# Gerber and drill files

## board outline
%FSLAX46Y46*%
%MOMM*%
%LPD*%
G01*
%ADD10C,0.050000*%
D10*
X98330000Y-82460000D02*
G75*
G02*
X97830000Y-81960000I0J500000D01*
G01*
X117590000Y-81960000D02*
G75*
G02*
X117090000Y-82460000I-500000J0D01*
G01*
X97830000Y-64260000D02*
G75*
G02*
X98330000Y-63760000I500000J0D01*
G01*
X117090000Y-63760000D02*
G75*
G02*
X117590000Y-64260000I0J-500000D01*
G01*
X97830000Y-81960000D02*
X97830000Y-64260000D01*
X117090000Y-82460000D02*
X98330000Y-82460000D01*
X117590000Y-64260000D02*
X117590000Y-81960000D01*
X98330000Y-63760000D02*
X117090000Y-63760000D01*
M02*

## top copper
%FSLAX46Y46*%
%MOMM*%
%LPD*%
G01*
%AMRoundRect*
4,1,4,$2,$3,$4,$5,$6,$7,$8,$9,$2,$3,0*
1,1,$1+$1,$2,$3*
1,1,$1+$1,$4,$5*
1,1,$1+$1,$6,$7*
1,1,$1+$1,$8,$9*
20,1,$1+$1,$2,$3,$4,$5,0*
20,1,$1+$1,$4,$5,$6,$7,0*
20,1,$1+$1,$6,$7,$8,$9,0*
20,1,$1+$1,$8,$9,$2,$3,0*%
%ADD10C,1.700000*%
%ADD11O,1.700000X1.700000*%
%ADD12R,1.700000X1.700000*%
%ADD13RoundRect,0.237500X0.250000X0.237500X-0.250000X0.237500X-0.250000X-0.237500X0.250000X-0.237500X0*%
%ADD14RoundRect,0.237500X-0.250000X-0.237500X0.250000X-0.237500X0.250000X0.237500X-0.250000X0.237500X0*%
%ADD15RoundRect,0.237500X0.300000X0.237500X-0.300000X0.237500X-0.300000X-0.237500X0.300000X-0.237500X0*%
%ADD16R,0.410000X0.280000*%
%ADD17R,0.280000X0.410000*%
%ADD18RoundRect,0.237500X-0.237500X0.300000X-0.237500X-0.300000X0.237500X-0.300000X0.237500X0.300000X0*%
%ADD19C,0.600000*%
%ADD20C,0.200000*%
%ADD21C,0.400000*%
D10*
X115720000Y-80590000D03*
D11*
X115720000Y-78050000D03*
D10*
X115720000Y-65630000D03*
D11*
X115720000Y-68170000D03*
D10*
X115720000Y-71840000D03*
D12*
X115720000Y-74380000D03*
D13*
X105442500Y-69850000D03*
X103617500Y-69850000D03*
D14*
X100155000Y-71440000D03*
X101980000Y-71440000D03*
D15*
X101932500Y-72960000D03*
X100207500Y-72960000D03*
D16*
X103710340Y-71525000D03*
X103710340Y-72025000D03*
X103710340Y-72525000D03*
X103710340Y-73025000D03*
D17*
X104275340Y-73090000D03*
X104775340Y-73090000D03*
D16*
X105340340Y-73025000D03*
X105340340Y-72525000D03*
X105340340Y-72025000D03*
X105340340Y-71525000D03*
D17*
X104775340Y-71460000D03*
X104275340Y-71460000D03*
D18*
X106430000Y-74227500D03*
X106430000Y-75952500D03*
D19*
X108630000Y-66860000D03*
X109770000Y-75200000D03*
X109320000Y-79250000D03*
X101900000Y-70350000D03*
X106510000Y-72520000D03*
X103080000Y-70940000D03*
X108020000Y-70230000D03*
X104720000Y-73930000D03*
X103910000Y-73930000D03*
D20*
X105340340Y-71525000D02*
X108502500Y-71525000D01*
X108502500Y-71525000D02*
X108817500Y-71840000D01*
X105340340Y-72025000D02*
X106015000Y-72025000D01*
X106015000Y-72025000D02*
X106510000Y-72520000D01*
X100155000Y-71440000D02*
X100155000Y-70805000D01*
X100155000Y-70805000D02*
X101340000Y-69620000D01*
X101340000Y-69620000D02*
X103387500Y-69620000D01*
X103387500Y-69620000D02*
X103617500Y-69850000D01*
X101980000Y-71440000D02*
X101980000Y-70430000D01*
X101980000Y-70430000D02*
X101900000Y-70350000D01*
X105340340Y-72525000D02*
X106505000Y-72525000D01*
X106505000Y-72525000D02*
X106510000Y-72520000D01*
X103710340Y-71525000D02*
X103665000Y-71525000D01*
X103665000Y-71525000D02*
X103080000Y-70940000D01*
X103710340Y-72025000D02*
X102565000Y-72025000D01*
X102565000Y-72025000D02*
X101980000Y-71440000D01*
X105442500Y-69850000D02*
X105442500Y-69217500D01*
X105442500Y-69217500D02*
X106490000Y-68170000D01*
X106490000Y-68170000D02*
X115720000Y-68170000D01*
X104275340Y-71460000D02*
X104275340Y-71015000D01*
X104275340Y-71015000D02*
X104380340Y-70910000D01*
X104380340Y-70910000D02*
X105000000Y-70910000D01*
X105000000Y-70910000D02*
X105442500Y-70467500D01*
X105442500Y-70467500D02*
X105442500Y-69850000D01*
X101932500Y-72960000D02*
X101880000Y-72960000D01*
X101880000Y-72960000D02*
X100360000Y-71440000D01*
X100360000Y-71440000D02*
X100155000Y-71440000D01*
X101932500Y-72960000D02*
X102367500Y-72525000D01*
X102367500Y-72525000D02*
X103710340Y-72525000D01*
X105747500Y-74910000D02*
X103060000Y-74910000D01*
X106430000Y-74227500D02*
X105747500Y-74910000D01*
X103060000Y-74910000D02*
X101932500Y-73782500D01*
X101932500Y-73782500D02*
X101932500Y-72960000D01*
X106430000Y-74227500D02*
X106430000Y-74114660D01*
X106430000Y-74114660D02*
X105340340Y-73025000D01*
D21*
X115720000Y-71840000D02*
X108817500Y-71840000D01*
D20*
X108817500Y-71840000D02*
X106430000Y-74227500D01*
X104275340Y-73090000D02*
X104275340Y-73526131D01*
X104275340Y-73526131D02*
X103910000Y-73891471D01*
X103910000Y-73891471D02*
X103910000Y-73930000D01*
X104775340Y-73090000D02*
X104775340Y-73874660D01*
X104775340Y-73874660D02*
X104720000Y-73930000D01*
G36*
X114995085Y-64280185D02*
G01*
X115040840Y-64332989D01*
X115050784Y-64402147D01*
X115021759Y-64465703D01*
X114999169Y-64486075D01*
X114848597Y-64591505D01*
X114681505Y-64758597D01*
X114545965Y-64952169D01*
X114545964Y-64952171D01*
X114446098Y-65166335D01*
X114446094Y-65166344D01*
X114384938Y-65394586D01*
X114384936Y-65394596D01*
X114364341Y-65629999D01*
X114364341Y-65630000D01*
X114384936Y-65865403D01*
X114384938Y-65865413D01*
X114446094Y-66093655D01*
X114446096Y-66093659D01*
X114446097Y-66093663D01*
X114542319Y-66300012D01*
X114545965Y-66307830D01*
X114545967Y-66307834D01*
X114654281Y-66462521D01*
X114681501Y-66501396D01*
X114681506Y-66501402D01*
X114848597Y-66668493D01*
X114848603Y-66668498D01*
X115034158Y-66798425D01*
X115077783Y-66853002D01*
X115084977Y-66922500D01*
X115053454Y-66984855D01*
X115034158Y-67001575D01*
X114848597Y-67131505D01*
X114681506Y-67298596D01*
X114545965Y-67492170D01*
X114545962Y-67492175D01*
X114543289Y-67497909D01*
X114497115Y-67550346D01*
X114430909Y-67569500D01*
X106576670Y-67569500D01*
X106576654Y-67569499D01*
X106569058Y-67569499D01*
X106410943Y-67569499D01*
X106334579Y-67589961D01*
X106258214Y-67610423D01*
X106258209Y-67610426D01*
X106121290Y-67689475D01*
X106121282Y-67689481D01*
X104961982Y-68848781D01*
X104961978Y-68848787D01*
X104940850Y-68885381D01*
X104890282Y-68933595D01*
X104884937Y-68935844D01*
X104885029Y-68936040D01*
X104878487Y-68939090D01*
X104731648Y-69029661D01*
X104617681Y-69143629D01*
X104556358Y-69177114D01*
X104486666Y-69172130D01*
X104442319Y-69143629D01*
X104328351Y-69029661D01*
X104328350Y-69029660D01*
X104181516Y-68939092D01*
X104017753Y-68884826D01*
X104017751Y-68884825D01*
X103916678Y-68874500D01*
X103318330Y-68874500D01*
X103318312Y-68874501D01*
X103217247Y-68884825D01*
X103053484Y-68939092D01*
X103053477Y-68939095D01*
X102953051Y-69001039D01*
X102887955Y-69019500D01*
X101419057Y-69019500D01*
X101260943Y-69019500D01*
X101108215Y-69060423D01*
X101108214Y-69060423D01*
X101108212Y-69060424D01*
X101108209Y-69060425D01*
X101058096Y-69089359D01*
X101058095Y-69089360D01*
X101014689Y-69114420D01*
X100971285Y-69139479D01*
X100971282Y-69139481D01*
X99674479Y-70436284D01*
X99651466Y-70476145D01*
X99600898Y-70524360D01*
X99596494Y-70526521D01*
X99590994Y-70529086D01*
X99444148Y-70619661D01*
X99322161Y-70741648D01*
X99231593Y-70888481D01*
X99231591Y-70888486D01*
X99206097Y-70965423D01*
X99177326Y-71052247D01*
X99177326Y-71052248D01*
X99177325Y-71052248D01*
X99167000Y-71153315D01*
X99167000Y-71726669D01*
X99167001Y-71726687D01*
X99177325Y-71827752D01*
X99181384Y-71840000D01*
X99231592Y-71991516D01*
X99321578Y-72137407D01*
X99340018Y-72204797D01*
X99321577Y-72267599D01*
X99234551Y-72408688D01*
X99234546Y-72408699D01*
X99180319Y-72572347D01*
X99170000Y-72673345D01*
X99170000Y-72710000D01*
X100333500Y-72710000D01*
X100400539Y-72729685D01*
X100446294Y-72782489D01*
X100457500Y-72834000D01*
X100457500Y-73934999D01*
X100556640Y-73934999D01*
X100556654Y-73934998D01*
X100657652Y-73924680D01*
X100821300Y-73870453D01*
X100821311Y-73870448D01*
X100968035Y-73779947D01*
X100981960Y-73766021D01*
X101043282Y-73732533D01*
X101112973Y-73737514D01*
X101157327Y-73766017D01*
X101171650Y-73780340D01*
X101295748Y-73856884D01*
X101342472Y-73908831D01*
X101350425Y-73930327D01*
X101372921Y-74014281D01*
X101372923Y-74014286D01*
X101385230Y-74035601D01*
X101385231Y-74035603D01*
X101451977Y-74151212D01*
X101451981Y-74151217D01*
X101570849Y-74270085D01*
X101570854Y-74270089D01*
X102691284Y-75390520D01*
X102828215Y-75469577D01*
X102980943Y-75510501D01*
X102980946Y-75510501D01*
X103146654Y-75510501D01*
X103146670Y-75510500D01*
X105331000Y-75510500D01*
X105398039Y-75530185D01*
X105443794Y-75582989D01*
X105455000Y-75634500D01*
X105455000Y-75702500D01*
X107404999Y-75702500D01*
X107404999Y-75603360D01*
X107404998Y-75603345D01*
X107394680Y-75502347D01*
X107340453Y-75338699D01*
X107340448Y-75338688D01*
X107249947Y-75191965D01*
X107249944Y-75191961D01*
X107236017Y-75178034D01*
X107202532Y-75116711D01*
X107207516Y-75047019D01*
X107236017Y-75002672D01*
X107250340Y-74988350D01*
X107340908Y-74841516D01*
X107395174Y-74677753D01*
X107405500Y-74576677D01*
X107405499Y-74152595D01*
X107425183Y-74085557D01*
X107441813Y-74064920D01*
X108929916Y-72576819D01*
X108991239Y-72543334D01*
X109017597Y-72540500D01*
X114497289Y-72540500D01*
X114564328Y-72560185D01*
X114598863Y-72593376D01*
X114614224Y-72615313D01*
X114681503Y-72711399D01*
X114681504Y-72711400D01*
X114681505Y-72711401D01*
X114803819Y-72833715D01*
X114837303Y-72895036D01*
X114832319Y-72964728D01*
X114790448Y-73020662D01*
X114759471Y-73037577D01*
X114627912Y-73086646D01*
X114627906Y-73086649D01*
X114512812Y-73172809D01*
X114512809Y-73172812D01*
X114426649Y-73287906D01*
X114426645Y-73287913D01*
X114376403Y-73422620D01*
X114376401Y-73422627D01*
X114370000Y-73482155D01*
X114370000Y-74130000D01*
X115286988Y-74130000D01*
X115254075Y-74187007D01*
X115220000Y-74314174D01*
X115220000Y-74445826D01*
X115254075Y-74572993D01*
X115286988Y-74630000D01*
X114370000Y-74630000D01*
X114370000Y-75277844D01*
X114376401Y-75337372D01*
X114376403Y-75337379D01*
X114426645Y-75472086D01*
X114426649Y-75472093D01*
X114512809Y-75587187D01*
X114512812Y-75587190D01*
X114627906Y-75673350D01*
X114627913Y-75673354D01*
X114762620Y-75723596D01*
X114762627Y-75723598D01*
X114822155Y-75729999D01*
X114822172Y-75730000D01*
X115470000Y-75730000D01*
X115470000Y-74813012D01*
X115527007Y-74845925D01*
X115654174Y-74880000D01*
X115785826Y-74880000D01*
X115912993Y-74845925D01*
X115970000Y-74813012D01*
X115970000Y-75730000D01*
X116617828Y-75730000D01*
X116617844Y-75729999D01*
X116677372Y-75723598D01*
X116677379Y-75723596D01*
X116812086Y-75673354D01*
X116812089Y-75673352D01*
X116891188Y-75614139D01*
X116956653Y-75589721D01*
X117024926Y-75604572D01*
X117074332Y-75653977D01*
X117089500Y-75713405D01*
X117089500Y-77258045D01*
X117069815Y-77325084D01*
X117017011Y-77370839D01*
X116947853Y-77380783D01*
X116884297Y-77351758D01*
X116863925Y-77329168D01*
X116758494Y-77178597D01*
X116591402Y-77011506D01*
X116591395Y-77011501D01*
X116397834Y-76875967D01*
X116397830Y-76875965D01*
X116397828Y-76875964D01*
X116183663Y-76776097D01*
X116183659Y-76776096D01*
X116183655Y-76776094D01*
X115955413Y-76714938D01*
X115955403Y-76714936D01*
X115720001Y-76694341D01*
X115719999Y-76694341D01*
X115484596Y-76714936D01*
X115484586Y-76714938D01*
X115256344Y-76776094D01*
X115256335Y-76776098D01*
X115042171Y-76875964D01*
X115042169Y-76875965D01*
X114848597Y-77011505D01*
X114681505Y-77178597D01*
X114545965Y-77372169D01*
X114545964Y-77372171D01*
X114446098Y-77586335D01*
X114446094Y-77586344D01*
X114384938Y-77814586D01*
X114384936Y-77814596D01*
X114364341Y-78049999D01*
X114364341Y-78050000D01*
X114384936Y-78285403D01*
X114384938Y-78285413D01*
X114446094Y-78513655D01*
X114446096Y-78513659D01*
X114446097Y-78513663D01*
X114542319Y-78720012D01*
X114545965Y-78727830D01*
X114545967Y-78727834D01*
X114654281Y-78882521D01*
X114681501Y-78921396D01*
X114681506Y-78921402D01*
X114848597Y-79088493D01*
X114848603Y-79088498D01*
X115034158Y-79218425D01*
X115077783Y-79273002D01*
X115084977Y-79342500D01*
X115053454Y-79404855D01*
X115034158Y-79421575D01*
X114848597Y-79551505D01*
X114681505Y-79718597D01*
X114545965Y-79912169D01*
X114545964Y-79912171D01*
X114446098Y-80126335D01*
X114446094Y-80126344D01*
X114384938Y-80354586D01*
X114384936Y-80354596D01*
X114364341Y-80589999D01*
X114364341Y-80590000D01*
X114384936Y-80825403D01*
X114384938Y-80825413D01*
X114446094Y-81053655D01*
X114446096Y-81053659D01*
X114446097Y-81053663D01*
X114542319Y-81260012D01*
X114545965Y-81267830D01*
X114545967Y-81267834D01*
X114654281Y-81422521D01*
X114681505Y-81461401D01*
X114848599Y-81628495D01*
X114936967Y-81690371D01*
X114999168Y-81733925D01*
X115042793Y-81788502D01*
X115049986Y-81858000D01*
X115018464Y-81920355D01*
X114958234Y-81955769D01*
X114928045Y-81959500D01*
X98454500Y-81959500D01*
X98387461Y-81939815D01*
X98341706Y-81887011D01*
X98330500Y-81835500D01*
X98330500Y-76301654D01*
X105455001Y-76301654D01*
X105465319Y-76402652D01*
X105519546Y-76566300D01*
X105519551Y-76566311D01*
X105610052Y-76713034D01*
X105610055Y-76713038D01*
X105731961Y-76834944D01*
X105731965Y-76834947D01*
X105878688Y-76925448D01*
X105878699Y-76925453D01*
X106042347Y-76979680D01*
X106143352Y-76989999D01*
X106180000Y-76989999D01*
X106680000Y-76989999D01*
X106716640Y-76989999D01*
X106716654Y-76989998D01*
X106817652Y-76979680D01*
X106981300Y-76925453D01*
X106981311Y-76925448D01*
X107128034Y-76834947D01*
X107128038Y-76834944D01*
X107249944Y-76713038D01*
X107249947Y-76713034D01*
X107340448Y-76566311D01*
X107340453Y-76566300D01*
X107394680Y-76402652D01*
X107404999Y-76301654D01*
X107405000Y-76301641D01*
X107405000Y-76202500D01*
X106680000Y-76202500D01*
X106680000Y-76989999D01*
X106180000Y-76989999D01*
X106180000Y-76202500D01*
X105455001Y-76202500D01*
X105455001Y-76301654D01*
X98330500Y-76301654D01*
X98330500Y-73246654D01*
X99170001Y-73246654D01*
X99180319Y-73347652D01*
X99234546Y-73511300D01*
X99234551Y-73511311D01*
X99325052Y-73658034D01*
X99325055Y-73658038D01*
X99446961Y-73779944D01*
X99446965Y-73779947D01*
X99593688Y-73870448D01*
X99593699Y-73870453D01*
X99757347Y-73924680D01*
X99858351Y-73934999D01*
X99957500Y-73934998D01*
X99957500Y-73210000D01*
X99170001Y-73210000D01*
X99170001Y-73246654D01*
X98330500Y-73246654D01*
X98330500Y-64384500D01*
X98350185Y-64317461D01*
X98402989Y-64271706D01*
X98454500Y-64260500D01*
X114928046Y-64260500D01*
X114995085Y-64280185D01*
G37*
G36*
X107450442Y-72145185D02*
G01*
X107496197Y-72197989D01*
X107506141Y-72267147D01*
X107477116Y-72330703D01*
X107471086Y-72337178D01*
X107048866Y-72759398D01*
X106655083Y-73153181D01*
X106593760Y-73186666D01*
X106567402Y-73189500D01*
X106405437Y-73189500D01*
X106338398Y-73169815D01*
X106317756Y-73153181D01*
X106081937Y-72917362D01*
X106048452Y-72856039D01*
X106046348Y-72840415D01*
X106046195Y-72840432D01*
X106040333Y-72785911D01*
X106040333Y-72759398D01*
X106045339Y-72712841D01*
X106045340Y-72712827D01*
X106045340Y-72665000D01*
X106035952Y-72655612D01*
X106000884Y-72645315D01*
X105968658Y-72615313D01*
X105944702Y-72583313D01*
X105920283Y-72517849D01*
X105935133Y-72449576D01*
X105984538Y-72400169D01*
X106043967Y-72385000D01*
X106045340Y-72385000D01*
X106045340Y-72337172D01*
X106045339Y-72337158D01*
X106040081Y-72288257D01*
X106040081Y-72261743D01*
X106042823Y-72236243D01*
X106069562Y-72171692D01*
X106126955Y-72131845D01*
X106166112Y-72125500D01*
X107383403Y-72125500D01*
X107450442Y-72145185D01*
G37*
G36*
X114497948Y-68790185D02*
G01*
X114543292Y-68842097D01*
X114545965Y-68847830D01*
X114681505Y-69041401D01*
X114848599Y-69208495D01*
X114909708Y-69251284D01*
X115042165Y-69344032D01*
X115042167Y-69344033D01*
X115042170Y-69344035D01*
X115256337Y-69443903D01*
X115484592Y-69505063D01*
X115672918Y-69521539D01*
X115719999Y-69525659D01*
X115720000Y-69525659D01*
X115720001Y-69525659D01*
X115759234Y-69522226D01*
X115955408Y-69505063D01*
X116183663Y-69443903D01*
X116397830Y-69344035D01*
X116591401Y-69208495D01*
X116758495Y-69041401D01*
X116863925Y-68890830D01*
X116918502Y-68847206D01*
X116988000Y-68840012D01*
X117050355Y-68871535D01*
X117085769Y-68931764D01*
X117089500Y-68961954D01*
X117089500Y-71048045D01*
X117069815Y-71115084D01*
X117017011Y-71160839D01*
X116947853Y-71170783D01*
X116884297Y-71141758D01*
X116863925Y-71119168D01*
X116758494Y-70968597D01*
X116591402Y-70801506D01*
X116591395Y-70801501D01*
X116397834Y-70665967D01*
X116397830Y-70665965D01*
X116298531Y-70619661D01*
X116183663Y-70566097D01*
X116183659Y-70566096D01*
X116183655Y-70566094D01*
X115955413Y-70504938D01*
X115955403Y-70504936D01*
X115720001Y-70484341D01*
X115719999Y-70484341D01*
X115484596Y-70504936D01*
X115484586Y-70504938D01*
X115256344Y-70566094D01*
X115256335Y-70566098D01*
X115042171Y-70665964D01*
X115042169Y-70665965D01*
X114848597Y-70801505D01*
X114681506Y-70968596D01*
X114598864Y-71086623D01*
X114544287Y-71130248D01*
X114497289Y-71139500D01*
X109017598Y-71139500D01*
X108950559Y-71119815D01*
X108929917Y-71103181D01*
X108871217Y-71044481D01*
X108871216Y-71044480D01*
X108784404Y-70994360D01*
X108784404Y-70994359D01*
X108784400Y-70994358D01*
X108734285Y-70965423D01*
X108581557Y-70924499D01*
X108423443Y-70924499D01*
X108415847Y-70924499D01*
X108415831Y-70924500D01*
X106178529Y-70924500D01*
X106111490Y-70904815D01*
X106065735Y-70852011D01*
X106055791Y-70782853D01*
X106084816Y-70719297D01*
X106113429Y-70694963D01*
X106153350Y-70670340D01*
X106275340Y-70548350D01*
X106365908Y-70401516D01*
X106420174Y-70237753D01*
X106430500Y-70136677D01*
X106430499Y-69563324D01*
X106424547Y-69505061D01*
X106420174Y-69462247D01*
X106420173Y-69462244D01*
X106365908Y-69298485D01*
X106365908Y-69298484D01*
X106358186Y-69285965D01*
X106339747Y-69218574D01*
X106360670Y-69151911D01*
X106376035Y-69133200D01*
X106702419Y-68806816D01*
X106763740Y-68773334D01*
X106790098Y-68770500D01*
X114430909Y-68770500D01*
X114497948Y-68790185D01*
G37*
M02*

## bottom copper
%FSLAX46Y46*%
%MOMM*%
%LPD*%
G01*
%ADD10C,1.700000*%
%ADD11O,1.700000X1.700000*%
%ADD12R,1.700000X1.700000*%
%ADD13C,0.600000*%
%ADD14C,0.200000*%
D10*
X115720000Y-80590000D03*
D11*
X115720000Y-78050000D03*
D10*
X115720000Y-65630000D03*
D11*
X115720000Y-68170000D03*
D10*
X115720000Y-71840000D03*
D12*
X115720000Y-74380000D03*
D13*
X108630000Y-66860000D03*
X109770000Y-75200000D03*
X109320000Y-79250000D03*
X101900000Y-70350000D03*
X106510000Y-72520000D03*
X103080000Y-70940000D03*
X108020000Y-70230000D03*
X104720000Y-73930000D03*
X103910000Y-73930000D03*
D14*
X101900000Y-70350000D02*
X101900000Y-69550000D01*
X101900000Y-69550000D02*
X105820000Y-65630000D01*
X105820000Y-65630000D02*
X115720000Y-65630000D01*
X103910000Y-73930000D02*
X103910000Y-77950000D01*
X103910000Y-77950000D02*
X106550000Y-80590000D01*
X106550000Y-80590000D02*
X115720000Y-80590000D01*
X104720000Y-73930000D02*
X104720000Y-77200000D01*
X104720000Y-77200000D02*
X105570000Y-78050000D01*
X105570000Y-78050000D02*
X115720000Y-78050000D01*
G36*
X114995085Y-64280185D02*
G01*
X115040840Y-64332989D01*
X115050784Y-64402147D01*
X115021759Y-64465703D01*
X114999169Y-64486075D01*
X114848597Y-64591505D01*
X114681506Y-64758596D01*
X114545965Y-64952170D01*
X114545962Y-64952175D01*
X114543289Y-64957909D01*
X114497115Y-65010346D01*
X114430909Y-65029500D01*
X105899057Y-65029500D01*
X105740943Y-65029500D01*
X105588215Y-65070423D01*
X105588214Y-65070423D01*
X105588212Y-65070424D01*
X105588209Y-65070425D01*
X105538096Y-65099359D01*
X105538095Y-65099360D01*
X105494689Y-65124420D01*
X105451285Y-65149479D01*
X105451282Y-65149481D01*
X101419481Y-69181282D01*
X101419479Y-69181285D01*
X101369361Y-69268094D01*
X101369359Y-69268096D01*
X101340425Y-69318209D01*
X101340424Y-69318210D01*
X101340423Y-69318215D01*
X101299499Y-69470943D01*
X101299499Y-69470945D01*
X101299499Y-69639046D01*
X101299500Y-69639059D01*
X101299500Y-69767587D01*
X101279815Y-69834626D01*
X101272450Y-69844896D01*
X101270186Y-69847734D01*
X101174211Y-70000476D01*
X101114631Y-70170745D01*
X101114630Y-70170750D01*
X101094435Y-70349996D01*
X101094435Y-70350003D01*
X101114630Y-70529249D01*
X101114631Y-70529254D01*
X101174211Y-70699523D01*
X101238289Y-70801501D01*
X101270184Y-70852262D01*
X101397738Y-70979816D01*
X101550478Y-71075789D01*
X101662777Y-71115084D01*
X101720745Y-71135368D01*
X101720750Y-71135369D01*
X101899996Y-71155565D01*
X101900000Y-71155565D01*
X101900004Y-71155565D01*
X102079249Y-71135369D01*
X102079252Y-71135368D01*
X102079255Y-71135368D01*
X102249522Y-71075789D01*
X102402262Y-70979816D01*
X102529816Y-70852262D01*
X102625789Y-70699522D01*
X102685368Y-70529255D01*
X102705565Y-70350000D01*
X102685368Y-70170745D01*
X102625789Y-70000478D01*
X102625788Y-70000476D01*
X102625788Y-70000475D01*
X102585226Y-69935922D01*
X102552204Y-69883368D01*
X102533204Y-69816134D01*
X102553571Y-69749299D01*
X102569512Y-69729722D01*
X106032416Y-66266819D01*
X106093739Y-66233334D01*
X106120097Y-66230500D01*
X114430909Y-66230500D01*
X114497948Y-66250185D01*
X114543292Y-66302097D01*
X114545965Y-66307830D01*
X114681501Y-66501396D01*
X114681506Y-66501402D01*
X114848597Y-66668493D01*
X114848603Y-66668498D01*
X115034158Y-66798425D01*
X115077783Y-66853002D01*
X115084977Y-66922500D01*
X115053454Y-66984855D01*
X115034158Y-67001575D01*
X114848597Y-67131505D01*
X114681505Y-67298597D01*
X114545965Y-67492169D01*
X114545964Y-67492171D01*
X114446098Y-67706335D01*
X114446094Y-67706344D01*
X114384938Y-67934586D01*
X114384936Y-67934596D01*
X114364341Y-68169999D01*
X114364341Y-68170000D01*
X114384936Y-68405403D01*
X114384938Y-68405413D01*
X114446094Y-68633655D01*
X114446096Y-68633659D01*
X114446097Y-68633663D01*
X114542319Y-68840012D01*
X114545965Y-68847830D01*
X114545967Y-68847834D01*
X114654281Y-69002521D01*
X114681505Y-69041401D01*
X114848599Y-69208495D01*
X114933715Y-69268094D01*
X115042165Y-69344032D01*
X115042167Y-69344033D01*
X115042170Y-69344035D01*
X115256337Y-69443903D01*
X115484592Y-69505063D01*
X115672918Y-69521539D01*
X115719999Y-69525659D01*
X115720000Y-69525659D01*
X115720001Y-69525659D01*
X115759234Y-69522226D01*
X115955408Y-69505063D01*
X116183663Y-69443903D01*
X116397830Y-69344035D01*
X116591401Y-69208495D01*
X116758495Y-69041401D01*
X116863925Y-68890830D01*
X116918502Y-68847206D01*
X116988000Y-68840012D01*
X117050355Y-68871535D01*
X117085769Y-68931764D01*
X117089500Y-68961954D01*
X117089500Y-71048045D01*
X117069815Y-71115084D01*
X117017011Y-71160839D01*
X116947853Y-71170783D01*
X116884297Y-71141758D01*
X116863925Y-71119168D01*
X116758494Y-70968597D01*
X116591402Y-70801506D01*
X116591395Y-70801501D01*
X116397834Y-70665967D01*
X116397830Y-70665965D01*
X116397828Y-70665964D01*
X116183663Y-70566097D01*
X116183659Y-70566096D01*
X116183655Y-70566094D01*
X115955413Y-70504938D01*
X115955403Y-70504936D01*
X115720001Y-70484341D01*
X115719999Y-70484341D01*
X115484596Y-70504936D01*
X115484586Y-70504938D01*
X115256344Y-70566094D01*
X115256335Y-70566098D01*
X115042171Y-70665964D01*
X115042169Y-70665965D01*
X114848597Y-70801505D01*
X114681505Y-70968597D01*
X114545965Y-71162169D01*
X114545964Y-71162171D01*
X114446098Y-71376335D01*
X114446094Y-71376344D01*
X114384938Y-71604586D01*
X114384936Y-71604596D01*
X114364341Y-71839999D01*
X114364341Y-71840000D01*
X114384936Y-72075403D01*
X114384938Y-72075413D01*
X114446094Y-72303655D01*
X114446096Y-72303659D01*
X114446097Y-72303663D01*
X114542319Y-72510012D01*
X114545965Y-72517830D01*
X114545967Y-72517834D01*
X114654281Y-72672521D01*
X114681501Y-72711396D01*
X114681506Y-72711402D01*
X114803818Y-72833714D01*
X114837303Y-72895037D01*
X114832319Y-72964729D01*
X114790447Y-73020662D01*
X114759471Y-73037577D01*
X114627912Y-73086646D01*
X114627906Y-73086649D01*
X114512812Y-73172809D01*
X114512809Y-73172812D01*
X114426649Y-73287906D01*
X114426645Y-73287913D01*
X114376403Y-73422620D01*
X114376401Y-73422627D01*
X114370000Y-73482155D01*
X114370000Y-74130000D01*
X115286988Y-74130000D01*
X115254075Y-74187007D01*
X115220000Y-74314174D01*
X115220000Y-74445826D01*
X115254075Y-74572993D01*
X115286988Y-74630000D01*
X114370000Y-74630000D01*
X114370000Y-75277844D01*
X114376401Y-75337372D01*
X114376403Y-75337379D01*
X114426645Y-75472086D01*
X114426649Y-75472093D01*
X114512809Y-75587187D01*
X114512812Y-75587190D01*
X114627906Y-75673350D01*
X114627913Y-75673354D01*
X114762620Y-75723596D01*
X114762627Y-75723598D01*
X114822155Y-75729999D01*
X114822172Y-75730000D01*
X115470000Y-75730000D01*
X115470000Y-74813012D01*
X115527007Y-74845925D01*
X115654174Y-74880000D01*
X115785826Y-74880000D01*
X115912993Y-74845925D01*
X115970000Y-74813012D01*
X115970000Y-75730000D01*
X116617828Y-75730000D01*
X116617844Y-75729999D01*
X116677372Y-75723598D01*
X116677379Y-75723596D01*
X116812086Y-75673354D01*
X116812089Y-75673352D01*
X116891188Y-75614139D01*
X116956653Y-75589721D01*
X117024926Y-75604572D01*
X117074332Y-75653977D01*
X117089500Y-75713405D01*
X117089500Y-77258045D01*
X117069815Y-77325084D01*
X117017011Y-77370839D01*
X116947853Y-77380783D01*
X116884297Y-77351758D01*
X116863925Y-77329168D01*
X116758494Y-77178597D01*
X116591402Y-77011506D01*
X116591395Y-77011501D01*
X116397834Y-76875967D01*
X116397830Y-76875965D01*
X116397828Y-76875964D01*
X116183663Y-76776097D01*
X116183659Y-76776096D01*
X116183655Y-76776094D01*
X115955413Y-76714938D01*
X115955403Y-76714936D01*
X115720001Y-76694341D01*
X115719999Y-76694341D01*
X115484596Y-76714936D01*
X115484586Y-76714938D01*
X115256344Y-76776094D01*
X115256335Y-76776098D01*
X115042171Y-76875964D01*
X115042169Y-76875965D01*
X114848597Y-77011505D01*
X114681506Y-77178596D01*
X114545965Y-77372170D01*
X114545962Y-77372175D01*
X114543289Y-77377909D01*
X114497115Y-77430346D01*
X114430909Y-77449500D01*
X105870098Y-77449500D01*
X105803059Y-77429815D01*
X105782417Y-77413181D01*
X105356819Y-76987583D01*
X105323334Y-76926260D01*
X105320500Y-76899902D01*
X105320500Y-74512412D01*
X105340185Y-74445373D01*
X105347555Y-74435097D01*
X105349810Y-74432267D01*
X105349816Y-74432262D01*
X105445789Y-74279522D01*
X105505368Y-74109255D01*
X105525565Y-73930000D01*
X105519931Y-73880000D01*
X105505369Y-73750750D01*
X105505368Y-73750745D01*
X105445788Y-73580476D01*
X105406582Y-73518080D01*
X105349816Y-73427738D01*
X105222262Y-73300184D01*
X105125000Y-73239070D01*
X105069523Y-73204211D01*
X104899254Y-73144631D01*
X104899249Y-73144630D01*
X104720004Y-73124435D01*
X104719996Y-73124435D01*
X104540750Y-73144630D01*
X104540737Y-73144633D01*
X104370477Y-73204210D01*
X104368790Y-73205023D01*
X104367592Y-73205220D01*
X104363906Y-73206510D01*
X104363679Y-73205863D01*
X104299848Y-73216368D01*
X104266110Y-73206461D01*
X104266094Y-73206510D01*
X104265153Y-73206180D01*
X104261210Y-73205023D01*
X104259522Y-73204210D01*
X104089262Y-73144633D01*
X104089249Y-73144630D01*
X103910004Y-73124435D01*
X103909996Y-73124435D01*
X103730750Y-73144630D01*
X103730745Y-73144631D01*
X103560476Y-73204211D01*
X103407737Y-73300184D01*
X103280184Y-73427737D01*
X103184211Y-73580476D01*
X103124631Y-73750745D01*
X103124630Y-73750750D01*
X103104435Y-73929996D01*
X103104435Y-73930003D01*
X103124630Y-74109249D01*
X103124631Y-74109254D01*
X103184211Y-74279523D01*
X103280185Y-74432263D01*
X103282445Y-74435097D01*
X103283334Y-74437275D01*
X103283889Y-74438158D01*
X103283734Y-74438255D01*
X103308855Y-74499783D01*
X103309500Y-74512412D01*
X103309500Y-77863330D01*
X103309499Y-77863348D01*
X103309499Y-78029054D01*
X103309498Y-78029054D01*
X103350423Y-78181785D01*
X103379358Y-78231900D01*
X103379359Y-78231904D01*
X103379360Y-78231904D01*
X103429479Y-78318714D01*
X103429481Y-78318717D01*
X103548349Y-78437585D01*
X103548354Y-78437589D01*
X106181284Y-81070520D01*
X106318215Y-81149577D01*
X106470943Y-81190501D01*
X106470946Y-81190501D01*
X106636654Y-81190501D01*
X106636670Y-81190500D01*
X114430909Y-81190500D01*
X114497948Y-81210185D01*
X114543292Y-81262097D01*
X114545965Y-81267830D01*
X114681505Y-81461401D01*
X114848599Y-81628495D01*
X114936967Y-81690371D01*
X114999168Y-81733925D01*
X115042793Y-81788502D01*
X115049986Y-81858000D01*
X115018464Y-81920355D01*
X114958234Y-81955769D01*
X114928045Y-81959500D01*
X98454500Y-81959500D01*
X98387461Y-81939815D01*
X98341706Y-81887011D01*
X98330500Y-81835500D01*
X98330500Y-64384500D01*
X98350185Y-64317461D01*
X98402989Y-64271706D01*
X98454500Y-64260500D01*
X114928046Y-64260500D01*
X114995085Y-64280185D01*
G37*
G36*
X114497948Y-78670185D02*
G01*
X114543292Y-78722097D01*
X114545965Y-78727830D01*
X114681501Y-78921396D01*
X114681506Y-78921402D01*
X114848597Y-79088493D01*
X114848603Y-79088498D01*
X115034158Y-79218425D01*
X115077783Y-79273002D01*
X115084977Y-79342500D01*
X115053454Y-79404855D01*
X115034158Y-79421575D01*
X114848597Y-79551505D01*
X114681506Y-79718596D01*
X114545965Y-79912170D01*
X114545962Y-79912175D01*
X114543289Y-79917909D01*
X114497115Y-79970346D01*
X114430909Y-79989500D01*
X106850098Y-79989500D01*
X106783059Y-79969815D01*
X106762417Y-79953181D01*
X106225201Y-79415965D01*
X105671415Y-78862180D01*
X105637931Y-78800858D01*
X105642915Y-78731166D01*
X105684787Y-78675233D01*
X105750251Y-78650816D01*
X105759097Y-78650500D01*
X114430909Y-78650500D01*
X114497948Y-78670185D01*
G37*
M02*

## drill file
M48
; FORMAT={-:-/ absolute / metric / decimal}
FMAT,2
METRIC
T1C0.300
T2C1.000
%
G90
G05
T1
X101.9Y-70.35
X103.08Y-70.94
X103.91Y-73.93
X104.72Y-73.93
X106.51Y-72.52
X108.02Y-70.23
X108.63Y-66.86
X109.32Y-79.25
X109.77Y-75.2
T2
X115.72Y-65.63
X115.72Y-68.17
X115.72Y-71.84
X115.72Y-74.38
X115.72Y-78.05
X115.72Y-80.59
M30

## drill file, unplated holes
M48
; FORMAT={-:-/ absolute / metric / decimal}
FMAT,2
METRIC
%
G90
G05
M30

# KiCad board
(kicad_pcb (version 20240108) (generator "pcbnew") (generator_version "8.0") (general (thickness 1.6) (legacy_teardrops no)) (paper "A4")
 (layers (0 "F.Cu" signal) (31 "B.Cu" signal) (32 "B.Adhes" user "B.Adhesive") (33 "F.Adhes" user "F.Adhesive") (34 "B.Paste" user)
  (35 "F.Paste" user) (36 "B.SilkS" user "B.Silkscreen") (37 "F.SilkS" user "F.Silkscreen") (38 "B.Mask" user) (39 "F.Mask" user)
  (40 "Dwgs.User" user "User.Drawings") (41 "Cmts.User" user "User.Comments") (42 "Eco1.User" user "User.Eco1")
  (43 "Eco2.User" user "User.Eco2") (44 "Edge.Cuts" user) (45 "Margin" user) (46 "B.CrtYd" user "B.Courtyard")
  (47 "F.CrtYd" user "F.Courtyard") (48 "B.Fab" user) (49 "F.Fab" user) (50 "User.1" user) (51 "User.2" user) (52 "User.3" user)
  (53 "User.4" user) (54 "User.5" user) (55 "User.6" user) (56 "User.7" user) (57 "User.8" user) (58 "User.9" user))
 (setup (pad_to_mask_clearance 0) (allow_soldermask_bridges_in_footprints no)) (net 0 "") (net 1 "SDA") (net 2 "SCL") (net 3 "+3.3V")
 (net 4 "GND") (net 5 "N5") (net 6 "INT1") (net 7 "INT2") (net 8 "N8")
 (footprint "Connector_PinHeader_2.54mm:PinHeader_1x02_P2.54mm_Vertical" (layer "F.Cu") (at 115.72 65.63)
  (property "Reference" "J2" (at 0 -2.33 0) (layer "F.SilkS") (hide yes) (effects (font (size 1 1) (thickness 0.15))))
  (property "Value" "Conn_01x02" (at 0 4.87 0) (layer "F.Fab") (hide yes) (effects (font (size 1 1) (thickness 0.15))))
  (pad "1" thru_hole circle (at 0 0) (size 1.7 1.7) (drill 1) (layers "*.Cu" "*.Mask") (remove_unused_layers no) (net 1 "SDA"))
  (pad "2" thru_hole oval (at 0 2.54) (size 1.7 1.7) (drill 1) (layers "*.Cu" "*.Mask") (remove_unused_layers no) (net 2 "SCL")))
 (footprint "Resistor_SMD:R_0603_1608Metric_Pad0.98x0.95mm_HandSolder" (layer "F.Cu") (at 104.53 69.85 180)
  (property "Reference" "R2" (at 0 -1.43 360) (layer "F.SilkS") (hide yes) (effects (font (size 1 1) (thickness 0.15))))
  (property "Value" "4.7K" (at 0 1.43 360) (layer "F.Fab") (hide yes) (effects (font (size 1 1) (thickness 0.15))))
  (pad "1" smd roundrect (at -0.9125 0 180) (size 0.975 0.95) (layers "F.Cu" "F.Paste" "F.Mask") (roundrect_rratio 0.25) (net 2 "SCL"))
  (pad "2" smd roundrect (at 0.9125 0 180) (size 0.975 0.95) (layers "F.Cu" "F.Paste" "F.Mask") (roundrect_rratio 0.25) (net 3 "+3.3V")))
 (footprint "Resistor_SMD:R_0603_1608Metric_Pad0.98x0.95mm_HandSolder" (layer "F.Cu") (at 101.0675 71.44)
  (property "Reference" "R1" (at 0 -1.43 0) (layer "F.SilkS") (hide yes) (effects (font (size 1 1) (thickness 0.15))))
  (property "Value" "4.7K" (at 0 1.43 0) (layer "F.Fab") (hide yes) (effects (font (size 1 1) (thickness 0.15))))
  (pad "1" smd roundrect (at -0.9125 0) (size 0.975 0.95) (layers "F.Cu" "F.Paste" "F.Mask") (roundrect_rratio 0.25) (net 3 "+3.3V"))
  (pad "2" smd roundrect (at 0.9125 0) (size 0.975 0.95) (layers "F.Cu" "F.Paste" "F.Mask") (roundrect_rratio 0.25) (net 1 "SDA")))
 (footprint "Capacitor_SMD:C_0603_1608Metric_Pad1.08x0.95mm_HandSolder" (layer "F.Cu") (at 101.07 72.96 180)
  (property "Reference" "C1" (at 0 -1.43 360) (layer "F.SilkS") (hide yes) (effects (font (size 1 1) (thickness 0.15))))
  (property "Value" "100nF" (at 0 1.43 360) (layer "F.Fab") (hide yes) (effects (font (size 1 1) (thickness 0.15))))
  (pad "1" smd roundrect (at -0.8625 0 180) (size 1.075 0.95) (layers "F.Cu" "F.Paste" "F.Mask") (roundrect_rratio 0.25) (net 3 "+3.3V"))
  (pad "2" smd roundrect (at 0.8625 0 180) (size 1.075 0.95) (layers "F.Cu" "F.Paste" "F.Mask") (roundrect_rratio 0.25) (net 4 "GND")))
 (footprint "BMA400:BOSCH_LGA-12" (layer "F.Cu") (at 104.52534 72.275)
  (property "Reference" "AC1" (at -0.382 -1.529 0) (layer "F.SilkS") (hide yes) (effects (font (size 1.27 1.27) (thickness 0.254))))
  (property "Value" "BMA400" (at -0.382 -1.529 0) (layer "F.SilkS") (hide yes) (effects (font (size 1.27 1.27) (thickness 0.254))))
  (pad "1" smd rect (at -0.815 -0.75 90) (size 0.28 0.41) (layers "F.Cu" "F.Paste" "F.Mask") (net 4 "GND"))
  (pad "2" smd rect (at -0.815 -0.25 90) (size 0.28 0.41) (layers "F.Cu" "F.Paste" "F.Mask") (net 1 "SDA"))
  (pad "3" smd rect (at -0.815 0.25 90) (size 0.28 0.41) (layers "F.Cu" "F.Paste" "F.Mask") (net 3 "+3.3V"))
  (pad "4" smd rect (at -0.815 0.75 90) (size 0.28 0.41) (layers "F.Cu" "F.Paste" "F.Mask") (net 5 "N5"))
  (pad "5" smd rect (at -0.25 0.815) (size 0.28 0.41) (layers "F.Cu" "F.Paste" "F.Mask") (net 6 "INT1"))
  (pad "6" smd rect (at 0.25 0.815) (size 0.28 0.41) (layers "F.Cu" "F.Paste" "F.Mask") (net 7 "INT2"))
  (pad "7" smd rect (at 0.815 0.75 90) (size 0.28 0.41) (layers "F.Cu" "F.Paste" "F.Mask") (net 3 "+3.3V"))
  (pad "8" smd rect (at 0.815 0.25 90) (size 0.28 0.41) (layers "F.Cu" "F.Paste" "F.Mask") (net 4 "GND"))
  (pad "9" smd rect (at 0.815 -0.25 90) (size 0.28 0.41) (layers "F.Cu" "F.Paste" "F.Mask") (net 4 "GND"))
  (pad "10" smd rect (at 0.815 -0.75 90) (size 0.28 0.41) (layers "F.Cu" "F.Paste" "F.Mask") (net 3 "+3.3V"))
  (pad "11" smd rect (at 0.25 -0.815) (size 0.28 0.41) (layers "F.Cu" "F.Paste" "F.Mask") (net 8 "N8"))
  (pad "12" smd rect (at -0.25 -0.815) (size 0.28 0.41) (layers "F.Cu" "F.Paste" "F.Mask") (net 2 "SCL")))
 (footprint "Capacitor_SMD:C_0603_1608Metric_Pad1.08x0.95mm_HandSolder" (layer "F.Cu") (at 106.43 75.09 -90)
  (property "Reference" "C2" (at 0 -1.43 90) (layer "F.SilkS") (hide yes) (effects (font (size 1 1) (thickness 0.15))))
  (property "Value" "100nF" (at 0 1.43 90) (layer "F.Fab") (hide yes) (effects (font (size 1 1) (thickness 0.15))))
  (pad "1" smd roundrect (at -0.8625 0 270) (size 1.075 0.95) (layers "F.Cu" "F.Paste" "F.Mask") (roundrect_rratio 0.25) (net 3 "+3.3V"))
  (pad "2" smd roundrect (at 0.8625 0 270) (size 1.075 0.95) (layers "F.Cu" "F.Paste" "F.Mask") (roundrect_rratio 0.25) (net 4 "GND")))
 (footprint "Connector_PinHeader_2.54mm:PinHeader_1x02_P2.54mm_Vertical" (layer "F.Cu") (at 115.72 71.84)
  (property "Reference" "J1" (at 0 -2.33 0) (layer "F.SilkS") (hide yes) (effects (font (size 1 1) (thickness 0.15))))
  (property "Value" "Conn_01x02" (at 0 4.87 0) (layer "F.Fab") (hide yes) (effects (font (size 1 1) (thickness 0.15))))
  (pad "1" thru_hole circle (at 0 0) (size 1.7 1.7) (drill 1) (layers "*.Cu" "*.Mask") (remove_unused_layers no) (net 3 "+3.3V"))
  (pad "2" thru_hole rect (at 0 2.54) (size 1.7 1.7) (drill 1) (layers "*.Cu" "*.Mask") (remove_unused_layers no) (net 4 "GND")))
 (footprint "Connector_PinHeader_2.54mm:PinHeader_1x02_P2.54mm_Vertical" (layer "F.Cu") (at 115.72 80.59 180)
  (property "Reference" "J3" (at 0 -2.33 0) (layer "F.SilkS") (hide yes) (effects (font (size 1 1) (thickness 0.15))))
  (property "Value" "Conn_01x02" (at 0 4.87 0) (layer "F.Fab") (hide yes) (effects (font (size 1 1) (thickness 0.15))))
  (pad "1" thru_hole circle (at 0 0 180) (size 1.7 1.7) (drill 1) (layers "*.Cu" "*.Mask") (remove_unused_layers no) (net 6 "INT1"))
  (pad "2" thru_hole oval (at 0 2.54 180) (size 1.7 1.7) (drill 1) (layers "*.Cu" "*.Mask") (remove_unused_layers no) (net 7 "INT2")))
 (gr_arc (start 117.09 63.76) (mid 117.443553 63.906447) (end 117.59 64.26) (stroke (width 0.05) (type default)) (layer "Edge.Cuts"))
 (gr_line (start 117.09 82.46) (end 98.33 82.46) (stroke (width 0.05) (type default)) (layer "Edge.Cuts"))
 (gr_arc (start 97.83 64.26) (mid 97.976447 63.906447) (end 98.33 63.76) (stroke (width 0.05) (type default)) (layer "Edge.Cuts"))
 (gr_arc (start 98.33 82.46) (mid 97.976447 82.313553) (end 97.83 81.96) (stroke (width 0.05) (type default)) (layer "Edge.Cuts"))
 (gr_arc (start 117.59 81.96) (mid 117.443553 82.313553) (end 117.09 82.46) (stroke (width 0.05) (type default)) (layer "Edge.Cuts"))
 (gr_line (start 117.59 64.26) (end 117.59 81.96) (stroke (width 0.05) (type default)) (layer "Edge.Cuts"))
 (gr_line (start 97.83 81.96) (end 97.83 64.26) (stroke (width 0.05) (type default)) (layer "Edge.Cuts"))
 (gr_line (start 98.33 63.76) (end 117.09 63.76) (stroke (width 0.05) (type default)) (layer "Edge.Cuts"))
 (segment (start 101.34 69.62) (end 103.3875 69.62) (width 0.2) (layer "F.Cu") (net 3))
 (segment (start 100.155 71.44) (end 100.155 70.805) (width 0.2) (layer "F.Cu") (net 3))
 (segment (start 108.5025 71.525) (end 108.8175 71.84) (width 0.2) (layer "F.Cu") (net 3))
 (segment (start 101.9325 73.7825) (end 101.9325 72.96) (width 0.2) (layer "F.Cu") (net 3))
 (segment (start 108.8175 71.84) (end 106.43 74.2275) (width 0.2) (layer "F.Cu") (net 3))
 (segment (start 106.43 74.2275) (end 106.43 74.11466) (width 0.2) (layer "F.Cu") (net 3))
 (segment (start 106.43 74.2275) (end 105.7475 74.91) (width 0.2) (layer "F.Cu") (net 3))
 (segment (start 102.3675 72.525) (end 103.71034 72.525) (width 0.2) (layer "F.Cu") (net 3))
 (segment (start 101.88 72.96) (end 100.36 71.44) (width 0.2) (layer "F.Cu") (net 3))
 (segment (start 106.43 74.11466) (end 105.34034 73.025) (width 0.2) (layer "F.Cu") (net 3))
 (segment (start 100.36 71.44) (end 100.155 71.44) (width 0.2) (layer "F.Cu") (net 3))
 (segment (start 101.9325 72.96) (end 102.3675 72.525) (width 0.2) (layer "F.Cu") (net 3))
 (segment (start 103.3875 69.62) (end 103.6175 69.85) (width 0.2) (layer "F.Cu") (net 3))
 (segment (start 105.34034 71.525) (end 108.5025 71.525) (width 0.2) (layer "F.Cu") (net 3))
 (segment (start 103.06 74.91) (end 101.9325 73.7825) (width 0.2) (layer "F.Cu") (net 3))
 (segment (start 101.9325 72.96) (end 101.88 72.96) (width 0.2) (layer "F.Cu") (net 3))
 (segment (start 115.72 71.84) (end 108.8175 71.84) (width 0.4) (layer "F.Cu") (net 3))
 (segment (start 105.7475 74.91) (end 103.06 74.91) (width 0.2) (layer "F.Cu") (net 3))
 (segment (start 100.155 70.805) (end 101.34 69.62) (width 0.2) (layer "F.Cu") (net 3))
 (segment (start 106.505 72.525) (end 106.51 72.52) (width 0.2) (layer "F.Cu") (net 4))
 (segment (start 103.71034 71.525) (end 103.665 71.525) (width 0.2) (layer "F.Cu") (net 4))
 (segment (start 103.665 71.525) (end 103.08 70.94) (width 0.2) (layer "F.Cu") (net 4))
 (segment (start 105.34034 72.525) (end 106.505 72.525) (width 0.2) (layer "F.Cu") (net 4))
 (segment (start 105.34034 72.025) (end 106.015 72.025) (width 0.2) (layer "F.Cu") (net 4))
 (segment (start 106.015 72.025) (end 106.51 72.52) (width 0.2) (layer "F.Cu") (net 4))
 (via (at 109.32 79.25) (size 0.6) (drill 0.3) (layers "F.Cu" "B.Cu") (free yes) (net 4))
 (via (at 108.02 70.23) (size 0.6) (drill 0.3) (layers "F.Cu" "B.Cu") (free yes) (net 4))
 (via (at 108.63 66.86) (size 0.6) (drill 0.3) (layers "F.Cu" "B.Cu") (free yes) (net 4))
 (via (at 103.08 70.94) (size 0.6) (drill 0.3) (layers "F.Cu" "B.Cu") (free yes) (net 4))
 (via (at 109.77 75.2) (size 0.6) (drill 0.3) (layers "F.Cu" "B.Cu") (free yes) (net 4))
 (via (at 106.51 72.52) (size 0.6) (drill 0.3) (layers "F.Cu" "B.Cu") (free yes) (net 4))
 (segment (start 104.77534 73.09) (end 104.77534 73.87466) (width 0.2) (layer "F.Cu") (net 7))
 (segment (start 104.77534 73.87466) (end 104.72 73.93) (width 0.2) (layer "F.Cu") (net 7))
 (via (at 104.72 73.93) (size 0.6) (drill 0.3) (layers "F.Cu" "B.Cu") (free yes) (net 7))
 (segment (start 104.72 73.93) (end 104.72 77.2) (width 0.2) (layer "B.Cu") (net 7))
 (segment (start 105.57 78.05) (end 115.72 78.05) (width 0.2) (layer "B.Cu") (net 7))
 (segment (start 104.72 77.2) (end 105.57 78.05) (width 0.2) (layer "B.Cu") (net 7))
 (segment (start 105 70.91) (end 105.4425 70.4675) (width 0.2) (layer "F.Cu") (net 2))
 (segment (start 105.4425 70.4675) (end 105.4425 69.85) (width 0.2) (layer "F.Cu") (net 2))
 (segment (start 105.4425 69.85) (end 105.4425 69.2175) (width 0.2) (layer "F.Cu") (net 2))
 (segment (start 106.49 68.17) (end 115.72 68.17) (width 0.2) (layer "F.Cu") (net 2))
 (segment (start 104.38034 70.91) (end 105 70.91) (width 0.2) (layer "F.Cu") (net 2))
 (segment (start 104.27534 71.015) (end 104.38034 70.91) (width 0.2) (layer "F.Cu") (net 2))
 (segment (start 104.27534 71.46) (end 104.27534 71.015) (width 0.2) (layer "F.Cu") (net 2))
 (segment (start 105.4425 69.2175) (end 106.49 68.17) (width 0.2) (layer "F.Cu") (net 2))
 (segment (start 103.91 73.891471) (end 103.91 73.93) (width 0.2) (layer "F.Cu") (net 6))
 (segment (start 104.27534 73.526131) (end 103.91 73.891471) (width 0.2) (layer "F.Cu") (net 6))
 (segment (start 104.27534 73.09) (end 104.27534 73.526131) (width 0.2) (layer "F.Cu") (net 6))
 (via (at 103.91 73.93) (size 0.6) (drill 0.3) (layers "F.Cu" "B.Cu") (free yes) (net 6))
 (segment (start 103.91 73.93) (end 103.91 77.95) (width 0.2) (layer "B.Cu") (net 6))
 (segment (start 106.55 80.59) (end 115.72 80.59) (width 0.2) (layer "B.Cu") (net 6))
 (segment (start 103.91 77.95) (end 106.55 80.59) (width 0.2) (layer "B.Cu") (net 6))
 (segment (start 101.98 70.43) (end 101.9 70.35) (width 0.2) (layer "F.Cu") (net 1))
 (segment (start 102.565 72.025) (end 101.98 71.44) (width 0.2) (layer "F.Cu") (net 1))
 (segment (start 101.98 71.44) (end 101.98 70.43) (width 0.2) (layer "F.Cu") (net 1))
 (segment (start 103.71034 72.025) (end 102.565 72.025) (width 0.2) (layer "F.Cu") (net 1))
 (via (at 101.9 70.35) (size 0.6) (drill 0.3) (layers "F.Cu" "B.Cu") (free yes) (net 1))
 (segment (start 101.9 70.35) (end 101.9 69.55) (width 0.2) (layer "B.Cu") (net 1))
 (segment (start 101.9 69.55) (end 105.82 65.63) (width 0.2) (layer "B.Cu") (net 1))
 (segment (start 105.82 65.63) (end 115.72 65.63) (width 0.2) (layer "B.Cu") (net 1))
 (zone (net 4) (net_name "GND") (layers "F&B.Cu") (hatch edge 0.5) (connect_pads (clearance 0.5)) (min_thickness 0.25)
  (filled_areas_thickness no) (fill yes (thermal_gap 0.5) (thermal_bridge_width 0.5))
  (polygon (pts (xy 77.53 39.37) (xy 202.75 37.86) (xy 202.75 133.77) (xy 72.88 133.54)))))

